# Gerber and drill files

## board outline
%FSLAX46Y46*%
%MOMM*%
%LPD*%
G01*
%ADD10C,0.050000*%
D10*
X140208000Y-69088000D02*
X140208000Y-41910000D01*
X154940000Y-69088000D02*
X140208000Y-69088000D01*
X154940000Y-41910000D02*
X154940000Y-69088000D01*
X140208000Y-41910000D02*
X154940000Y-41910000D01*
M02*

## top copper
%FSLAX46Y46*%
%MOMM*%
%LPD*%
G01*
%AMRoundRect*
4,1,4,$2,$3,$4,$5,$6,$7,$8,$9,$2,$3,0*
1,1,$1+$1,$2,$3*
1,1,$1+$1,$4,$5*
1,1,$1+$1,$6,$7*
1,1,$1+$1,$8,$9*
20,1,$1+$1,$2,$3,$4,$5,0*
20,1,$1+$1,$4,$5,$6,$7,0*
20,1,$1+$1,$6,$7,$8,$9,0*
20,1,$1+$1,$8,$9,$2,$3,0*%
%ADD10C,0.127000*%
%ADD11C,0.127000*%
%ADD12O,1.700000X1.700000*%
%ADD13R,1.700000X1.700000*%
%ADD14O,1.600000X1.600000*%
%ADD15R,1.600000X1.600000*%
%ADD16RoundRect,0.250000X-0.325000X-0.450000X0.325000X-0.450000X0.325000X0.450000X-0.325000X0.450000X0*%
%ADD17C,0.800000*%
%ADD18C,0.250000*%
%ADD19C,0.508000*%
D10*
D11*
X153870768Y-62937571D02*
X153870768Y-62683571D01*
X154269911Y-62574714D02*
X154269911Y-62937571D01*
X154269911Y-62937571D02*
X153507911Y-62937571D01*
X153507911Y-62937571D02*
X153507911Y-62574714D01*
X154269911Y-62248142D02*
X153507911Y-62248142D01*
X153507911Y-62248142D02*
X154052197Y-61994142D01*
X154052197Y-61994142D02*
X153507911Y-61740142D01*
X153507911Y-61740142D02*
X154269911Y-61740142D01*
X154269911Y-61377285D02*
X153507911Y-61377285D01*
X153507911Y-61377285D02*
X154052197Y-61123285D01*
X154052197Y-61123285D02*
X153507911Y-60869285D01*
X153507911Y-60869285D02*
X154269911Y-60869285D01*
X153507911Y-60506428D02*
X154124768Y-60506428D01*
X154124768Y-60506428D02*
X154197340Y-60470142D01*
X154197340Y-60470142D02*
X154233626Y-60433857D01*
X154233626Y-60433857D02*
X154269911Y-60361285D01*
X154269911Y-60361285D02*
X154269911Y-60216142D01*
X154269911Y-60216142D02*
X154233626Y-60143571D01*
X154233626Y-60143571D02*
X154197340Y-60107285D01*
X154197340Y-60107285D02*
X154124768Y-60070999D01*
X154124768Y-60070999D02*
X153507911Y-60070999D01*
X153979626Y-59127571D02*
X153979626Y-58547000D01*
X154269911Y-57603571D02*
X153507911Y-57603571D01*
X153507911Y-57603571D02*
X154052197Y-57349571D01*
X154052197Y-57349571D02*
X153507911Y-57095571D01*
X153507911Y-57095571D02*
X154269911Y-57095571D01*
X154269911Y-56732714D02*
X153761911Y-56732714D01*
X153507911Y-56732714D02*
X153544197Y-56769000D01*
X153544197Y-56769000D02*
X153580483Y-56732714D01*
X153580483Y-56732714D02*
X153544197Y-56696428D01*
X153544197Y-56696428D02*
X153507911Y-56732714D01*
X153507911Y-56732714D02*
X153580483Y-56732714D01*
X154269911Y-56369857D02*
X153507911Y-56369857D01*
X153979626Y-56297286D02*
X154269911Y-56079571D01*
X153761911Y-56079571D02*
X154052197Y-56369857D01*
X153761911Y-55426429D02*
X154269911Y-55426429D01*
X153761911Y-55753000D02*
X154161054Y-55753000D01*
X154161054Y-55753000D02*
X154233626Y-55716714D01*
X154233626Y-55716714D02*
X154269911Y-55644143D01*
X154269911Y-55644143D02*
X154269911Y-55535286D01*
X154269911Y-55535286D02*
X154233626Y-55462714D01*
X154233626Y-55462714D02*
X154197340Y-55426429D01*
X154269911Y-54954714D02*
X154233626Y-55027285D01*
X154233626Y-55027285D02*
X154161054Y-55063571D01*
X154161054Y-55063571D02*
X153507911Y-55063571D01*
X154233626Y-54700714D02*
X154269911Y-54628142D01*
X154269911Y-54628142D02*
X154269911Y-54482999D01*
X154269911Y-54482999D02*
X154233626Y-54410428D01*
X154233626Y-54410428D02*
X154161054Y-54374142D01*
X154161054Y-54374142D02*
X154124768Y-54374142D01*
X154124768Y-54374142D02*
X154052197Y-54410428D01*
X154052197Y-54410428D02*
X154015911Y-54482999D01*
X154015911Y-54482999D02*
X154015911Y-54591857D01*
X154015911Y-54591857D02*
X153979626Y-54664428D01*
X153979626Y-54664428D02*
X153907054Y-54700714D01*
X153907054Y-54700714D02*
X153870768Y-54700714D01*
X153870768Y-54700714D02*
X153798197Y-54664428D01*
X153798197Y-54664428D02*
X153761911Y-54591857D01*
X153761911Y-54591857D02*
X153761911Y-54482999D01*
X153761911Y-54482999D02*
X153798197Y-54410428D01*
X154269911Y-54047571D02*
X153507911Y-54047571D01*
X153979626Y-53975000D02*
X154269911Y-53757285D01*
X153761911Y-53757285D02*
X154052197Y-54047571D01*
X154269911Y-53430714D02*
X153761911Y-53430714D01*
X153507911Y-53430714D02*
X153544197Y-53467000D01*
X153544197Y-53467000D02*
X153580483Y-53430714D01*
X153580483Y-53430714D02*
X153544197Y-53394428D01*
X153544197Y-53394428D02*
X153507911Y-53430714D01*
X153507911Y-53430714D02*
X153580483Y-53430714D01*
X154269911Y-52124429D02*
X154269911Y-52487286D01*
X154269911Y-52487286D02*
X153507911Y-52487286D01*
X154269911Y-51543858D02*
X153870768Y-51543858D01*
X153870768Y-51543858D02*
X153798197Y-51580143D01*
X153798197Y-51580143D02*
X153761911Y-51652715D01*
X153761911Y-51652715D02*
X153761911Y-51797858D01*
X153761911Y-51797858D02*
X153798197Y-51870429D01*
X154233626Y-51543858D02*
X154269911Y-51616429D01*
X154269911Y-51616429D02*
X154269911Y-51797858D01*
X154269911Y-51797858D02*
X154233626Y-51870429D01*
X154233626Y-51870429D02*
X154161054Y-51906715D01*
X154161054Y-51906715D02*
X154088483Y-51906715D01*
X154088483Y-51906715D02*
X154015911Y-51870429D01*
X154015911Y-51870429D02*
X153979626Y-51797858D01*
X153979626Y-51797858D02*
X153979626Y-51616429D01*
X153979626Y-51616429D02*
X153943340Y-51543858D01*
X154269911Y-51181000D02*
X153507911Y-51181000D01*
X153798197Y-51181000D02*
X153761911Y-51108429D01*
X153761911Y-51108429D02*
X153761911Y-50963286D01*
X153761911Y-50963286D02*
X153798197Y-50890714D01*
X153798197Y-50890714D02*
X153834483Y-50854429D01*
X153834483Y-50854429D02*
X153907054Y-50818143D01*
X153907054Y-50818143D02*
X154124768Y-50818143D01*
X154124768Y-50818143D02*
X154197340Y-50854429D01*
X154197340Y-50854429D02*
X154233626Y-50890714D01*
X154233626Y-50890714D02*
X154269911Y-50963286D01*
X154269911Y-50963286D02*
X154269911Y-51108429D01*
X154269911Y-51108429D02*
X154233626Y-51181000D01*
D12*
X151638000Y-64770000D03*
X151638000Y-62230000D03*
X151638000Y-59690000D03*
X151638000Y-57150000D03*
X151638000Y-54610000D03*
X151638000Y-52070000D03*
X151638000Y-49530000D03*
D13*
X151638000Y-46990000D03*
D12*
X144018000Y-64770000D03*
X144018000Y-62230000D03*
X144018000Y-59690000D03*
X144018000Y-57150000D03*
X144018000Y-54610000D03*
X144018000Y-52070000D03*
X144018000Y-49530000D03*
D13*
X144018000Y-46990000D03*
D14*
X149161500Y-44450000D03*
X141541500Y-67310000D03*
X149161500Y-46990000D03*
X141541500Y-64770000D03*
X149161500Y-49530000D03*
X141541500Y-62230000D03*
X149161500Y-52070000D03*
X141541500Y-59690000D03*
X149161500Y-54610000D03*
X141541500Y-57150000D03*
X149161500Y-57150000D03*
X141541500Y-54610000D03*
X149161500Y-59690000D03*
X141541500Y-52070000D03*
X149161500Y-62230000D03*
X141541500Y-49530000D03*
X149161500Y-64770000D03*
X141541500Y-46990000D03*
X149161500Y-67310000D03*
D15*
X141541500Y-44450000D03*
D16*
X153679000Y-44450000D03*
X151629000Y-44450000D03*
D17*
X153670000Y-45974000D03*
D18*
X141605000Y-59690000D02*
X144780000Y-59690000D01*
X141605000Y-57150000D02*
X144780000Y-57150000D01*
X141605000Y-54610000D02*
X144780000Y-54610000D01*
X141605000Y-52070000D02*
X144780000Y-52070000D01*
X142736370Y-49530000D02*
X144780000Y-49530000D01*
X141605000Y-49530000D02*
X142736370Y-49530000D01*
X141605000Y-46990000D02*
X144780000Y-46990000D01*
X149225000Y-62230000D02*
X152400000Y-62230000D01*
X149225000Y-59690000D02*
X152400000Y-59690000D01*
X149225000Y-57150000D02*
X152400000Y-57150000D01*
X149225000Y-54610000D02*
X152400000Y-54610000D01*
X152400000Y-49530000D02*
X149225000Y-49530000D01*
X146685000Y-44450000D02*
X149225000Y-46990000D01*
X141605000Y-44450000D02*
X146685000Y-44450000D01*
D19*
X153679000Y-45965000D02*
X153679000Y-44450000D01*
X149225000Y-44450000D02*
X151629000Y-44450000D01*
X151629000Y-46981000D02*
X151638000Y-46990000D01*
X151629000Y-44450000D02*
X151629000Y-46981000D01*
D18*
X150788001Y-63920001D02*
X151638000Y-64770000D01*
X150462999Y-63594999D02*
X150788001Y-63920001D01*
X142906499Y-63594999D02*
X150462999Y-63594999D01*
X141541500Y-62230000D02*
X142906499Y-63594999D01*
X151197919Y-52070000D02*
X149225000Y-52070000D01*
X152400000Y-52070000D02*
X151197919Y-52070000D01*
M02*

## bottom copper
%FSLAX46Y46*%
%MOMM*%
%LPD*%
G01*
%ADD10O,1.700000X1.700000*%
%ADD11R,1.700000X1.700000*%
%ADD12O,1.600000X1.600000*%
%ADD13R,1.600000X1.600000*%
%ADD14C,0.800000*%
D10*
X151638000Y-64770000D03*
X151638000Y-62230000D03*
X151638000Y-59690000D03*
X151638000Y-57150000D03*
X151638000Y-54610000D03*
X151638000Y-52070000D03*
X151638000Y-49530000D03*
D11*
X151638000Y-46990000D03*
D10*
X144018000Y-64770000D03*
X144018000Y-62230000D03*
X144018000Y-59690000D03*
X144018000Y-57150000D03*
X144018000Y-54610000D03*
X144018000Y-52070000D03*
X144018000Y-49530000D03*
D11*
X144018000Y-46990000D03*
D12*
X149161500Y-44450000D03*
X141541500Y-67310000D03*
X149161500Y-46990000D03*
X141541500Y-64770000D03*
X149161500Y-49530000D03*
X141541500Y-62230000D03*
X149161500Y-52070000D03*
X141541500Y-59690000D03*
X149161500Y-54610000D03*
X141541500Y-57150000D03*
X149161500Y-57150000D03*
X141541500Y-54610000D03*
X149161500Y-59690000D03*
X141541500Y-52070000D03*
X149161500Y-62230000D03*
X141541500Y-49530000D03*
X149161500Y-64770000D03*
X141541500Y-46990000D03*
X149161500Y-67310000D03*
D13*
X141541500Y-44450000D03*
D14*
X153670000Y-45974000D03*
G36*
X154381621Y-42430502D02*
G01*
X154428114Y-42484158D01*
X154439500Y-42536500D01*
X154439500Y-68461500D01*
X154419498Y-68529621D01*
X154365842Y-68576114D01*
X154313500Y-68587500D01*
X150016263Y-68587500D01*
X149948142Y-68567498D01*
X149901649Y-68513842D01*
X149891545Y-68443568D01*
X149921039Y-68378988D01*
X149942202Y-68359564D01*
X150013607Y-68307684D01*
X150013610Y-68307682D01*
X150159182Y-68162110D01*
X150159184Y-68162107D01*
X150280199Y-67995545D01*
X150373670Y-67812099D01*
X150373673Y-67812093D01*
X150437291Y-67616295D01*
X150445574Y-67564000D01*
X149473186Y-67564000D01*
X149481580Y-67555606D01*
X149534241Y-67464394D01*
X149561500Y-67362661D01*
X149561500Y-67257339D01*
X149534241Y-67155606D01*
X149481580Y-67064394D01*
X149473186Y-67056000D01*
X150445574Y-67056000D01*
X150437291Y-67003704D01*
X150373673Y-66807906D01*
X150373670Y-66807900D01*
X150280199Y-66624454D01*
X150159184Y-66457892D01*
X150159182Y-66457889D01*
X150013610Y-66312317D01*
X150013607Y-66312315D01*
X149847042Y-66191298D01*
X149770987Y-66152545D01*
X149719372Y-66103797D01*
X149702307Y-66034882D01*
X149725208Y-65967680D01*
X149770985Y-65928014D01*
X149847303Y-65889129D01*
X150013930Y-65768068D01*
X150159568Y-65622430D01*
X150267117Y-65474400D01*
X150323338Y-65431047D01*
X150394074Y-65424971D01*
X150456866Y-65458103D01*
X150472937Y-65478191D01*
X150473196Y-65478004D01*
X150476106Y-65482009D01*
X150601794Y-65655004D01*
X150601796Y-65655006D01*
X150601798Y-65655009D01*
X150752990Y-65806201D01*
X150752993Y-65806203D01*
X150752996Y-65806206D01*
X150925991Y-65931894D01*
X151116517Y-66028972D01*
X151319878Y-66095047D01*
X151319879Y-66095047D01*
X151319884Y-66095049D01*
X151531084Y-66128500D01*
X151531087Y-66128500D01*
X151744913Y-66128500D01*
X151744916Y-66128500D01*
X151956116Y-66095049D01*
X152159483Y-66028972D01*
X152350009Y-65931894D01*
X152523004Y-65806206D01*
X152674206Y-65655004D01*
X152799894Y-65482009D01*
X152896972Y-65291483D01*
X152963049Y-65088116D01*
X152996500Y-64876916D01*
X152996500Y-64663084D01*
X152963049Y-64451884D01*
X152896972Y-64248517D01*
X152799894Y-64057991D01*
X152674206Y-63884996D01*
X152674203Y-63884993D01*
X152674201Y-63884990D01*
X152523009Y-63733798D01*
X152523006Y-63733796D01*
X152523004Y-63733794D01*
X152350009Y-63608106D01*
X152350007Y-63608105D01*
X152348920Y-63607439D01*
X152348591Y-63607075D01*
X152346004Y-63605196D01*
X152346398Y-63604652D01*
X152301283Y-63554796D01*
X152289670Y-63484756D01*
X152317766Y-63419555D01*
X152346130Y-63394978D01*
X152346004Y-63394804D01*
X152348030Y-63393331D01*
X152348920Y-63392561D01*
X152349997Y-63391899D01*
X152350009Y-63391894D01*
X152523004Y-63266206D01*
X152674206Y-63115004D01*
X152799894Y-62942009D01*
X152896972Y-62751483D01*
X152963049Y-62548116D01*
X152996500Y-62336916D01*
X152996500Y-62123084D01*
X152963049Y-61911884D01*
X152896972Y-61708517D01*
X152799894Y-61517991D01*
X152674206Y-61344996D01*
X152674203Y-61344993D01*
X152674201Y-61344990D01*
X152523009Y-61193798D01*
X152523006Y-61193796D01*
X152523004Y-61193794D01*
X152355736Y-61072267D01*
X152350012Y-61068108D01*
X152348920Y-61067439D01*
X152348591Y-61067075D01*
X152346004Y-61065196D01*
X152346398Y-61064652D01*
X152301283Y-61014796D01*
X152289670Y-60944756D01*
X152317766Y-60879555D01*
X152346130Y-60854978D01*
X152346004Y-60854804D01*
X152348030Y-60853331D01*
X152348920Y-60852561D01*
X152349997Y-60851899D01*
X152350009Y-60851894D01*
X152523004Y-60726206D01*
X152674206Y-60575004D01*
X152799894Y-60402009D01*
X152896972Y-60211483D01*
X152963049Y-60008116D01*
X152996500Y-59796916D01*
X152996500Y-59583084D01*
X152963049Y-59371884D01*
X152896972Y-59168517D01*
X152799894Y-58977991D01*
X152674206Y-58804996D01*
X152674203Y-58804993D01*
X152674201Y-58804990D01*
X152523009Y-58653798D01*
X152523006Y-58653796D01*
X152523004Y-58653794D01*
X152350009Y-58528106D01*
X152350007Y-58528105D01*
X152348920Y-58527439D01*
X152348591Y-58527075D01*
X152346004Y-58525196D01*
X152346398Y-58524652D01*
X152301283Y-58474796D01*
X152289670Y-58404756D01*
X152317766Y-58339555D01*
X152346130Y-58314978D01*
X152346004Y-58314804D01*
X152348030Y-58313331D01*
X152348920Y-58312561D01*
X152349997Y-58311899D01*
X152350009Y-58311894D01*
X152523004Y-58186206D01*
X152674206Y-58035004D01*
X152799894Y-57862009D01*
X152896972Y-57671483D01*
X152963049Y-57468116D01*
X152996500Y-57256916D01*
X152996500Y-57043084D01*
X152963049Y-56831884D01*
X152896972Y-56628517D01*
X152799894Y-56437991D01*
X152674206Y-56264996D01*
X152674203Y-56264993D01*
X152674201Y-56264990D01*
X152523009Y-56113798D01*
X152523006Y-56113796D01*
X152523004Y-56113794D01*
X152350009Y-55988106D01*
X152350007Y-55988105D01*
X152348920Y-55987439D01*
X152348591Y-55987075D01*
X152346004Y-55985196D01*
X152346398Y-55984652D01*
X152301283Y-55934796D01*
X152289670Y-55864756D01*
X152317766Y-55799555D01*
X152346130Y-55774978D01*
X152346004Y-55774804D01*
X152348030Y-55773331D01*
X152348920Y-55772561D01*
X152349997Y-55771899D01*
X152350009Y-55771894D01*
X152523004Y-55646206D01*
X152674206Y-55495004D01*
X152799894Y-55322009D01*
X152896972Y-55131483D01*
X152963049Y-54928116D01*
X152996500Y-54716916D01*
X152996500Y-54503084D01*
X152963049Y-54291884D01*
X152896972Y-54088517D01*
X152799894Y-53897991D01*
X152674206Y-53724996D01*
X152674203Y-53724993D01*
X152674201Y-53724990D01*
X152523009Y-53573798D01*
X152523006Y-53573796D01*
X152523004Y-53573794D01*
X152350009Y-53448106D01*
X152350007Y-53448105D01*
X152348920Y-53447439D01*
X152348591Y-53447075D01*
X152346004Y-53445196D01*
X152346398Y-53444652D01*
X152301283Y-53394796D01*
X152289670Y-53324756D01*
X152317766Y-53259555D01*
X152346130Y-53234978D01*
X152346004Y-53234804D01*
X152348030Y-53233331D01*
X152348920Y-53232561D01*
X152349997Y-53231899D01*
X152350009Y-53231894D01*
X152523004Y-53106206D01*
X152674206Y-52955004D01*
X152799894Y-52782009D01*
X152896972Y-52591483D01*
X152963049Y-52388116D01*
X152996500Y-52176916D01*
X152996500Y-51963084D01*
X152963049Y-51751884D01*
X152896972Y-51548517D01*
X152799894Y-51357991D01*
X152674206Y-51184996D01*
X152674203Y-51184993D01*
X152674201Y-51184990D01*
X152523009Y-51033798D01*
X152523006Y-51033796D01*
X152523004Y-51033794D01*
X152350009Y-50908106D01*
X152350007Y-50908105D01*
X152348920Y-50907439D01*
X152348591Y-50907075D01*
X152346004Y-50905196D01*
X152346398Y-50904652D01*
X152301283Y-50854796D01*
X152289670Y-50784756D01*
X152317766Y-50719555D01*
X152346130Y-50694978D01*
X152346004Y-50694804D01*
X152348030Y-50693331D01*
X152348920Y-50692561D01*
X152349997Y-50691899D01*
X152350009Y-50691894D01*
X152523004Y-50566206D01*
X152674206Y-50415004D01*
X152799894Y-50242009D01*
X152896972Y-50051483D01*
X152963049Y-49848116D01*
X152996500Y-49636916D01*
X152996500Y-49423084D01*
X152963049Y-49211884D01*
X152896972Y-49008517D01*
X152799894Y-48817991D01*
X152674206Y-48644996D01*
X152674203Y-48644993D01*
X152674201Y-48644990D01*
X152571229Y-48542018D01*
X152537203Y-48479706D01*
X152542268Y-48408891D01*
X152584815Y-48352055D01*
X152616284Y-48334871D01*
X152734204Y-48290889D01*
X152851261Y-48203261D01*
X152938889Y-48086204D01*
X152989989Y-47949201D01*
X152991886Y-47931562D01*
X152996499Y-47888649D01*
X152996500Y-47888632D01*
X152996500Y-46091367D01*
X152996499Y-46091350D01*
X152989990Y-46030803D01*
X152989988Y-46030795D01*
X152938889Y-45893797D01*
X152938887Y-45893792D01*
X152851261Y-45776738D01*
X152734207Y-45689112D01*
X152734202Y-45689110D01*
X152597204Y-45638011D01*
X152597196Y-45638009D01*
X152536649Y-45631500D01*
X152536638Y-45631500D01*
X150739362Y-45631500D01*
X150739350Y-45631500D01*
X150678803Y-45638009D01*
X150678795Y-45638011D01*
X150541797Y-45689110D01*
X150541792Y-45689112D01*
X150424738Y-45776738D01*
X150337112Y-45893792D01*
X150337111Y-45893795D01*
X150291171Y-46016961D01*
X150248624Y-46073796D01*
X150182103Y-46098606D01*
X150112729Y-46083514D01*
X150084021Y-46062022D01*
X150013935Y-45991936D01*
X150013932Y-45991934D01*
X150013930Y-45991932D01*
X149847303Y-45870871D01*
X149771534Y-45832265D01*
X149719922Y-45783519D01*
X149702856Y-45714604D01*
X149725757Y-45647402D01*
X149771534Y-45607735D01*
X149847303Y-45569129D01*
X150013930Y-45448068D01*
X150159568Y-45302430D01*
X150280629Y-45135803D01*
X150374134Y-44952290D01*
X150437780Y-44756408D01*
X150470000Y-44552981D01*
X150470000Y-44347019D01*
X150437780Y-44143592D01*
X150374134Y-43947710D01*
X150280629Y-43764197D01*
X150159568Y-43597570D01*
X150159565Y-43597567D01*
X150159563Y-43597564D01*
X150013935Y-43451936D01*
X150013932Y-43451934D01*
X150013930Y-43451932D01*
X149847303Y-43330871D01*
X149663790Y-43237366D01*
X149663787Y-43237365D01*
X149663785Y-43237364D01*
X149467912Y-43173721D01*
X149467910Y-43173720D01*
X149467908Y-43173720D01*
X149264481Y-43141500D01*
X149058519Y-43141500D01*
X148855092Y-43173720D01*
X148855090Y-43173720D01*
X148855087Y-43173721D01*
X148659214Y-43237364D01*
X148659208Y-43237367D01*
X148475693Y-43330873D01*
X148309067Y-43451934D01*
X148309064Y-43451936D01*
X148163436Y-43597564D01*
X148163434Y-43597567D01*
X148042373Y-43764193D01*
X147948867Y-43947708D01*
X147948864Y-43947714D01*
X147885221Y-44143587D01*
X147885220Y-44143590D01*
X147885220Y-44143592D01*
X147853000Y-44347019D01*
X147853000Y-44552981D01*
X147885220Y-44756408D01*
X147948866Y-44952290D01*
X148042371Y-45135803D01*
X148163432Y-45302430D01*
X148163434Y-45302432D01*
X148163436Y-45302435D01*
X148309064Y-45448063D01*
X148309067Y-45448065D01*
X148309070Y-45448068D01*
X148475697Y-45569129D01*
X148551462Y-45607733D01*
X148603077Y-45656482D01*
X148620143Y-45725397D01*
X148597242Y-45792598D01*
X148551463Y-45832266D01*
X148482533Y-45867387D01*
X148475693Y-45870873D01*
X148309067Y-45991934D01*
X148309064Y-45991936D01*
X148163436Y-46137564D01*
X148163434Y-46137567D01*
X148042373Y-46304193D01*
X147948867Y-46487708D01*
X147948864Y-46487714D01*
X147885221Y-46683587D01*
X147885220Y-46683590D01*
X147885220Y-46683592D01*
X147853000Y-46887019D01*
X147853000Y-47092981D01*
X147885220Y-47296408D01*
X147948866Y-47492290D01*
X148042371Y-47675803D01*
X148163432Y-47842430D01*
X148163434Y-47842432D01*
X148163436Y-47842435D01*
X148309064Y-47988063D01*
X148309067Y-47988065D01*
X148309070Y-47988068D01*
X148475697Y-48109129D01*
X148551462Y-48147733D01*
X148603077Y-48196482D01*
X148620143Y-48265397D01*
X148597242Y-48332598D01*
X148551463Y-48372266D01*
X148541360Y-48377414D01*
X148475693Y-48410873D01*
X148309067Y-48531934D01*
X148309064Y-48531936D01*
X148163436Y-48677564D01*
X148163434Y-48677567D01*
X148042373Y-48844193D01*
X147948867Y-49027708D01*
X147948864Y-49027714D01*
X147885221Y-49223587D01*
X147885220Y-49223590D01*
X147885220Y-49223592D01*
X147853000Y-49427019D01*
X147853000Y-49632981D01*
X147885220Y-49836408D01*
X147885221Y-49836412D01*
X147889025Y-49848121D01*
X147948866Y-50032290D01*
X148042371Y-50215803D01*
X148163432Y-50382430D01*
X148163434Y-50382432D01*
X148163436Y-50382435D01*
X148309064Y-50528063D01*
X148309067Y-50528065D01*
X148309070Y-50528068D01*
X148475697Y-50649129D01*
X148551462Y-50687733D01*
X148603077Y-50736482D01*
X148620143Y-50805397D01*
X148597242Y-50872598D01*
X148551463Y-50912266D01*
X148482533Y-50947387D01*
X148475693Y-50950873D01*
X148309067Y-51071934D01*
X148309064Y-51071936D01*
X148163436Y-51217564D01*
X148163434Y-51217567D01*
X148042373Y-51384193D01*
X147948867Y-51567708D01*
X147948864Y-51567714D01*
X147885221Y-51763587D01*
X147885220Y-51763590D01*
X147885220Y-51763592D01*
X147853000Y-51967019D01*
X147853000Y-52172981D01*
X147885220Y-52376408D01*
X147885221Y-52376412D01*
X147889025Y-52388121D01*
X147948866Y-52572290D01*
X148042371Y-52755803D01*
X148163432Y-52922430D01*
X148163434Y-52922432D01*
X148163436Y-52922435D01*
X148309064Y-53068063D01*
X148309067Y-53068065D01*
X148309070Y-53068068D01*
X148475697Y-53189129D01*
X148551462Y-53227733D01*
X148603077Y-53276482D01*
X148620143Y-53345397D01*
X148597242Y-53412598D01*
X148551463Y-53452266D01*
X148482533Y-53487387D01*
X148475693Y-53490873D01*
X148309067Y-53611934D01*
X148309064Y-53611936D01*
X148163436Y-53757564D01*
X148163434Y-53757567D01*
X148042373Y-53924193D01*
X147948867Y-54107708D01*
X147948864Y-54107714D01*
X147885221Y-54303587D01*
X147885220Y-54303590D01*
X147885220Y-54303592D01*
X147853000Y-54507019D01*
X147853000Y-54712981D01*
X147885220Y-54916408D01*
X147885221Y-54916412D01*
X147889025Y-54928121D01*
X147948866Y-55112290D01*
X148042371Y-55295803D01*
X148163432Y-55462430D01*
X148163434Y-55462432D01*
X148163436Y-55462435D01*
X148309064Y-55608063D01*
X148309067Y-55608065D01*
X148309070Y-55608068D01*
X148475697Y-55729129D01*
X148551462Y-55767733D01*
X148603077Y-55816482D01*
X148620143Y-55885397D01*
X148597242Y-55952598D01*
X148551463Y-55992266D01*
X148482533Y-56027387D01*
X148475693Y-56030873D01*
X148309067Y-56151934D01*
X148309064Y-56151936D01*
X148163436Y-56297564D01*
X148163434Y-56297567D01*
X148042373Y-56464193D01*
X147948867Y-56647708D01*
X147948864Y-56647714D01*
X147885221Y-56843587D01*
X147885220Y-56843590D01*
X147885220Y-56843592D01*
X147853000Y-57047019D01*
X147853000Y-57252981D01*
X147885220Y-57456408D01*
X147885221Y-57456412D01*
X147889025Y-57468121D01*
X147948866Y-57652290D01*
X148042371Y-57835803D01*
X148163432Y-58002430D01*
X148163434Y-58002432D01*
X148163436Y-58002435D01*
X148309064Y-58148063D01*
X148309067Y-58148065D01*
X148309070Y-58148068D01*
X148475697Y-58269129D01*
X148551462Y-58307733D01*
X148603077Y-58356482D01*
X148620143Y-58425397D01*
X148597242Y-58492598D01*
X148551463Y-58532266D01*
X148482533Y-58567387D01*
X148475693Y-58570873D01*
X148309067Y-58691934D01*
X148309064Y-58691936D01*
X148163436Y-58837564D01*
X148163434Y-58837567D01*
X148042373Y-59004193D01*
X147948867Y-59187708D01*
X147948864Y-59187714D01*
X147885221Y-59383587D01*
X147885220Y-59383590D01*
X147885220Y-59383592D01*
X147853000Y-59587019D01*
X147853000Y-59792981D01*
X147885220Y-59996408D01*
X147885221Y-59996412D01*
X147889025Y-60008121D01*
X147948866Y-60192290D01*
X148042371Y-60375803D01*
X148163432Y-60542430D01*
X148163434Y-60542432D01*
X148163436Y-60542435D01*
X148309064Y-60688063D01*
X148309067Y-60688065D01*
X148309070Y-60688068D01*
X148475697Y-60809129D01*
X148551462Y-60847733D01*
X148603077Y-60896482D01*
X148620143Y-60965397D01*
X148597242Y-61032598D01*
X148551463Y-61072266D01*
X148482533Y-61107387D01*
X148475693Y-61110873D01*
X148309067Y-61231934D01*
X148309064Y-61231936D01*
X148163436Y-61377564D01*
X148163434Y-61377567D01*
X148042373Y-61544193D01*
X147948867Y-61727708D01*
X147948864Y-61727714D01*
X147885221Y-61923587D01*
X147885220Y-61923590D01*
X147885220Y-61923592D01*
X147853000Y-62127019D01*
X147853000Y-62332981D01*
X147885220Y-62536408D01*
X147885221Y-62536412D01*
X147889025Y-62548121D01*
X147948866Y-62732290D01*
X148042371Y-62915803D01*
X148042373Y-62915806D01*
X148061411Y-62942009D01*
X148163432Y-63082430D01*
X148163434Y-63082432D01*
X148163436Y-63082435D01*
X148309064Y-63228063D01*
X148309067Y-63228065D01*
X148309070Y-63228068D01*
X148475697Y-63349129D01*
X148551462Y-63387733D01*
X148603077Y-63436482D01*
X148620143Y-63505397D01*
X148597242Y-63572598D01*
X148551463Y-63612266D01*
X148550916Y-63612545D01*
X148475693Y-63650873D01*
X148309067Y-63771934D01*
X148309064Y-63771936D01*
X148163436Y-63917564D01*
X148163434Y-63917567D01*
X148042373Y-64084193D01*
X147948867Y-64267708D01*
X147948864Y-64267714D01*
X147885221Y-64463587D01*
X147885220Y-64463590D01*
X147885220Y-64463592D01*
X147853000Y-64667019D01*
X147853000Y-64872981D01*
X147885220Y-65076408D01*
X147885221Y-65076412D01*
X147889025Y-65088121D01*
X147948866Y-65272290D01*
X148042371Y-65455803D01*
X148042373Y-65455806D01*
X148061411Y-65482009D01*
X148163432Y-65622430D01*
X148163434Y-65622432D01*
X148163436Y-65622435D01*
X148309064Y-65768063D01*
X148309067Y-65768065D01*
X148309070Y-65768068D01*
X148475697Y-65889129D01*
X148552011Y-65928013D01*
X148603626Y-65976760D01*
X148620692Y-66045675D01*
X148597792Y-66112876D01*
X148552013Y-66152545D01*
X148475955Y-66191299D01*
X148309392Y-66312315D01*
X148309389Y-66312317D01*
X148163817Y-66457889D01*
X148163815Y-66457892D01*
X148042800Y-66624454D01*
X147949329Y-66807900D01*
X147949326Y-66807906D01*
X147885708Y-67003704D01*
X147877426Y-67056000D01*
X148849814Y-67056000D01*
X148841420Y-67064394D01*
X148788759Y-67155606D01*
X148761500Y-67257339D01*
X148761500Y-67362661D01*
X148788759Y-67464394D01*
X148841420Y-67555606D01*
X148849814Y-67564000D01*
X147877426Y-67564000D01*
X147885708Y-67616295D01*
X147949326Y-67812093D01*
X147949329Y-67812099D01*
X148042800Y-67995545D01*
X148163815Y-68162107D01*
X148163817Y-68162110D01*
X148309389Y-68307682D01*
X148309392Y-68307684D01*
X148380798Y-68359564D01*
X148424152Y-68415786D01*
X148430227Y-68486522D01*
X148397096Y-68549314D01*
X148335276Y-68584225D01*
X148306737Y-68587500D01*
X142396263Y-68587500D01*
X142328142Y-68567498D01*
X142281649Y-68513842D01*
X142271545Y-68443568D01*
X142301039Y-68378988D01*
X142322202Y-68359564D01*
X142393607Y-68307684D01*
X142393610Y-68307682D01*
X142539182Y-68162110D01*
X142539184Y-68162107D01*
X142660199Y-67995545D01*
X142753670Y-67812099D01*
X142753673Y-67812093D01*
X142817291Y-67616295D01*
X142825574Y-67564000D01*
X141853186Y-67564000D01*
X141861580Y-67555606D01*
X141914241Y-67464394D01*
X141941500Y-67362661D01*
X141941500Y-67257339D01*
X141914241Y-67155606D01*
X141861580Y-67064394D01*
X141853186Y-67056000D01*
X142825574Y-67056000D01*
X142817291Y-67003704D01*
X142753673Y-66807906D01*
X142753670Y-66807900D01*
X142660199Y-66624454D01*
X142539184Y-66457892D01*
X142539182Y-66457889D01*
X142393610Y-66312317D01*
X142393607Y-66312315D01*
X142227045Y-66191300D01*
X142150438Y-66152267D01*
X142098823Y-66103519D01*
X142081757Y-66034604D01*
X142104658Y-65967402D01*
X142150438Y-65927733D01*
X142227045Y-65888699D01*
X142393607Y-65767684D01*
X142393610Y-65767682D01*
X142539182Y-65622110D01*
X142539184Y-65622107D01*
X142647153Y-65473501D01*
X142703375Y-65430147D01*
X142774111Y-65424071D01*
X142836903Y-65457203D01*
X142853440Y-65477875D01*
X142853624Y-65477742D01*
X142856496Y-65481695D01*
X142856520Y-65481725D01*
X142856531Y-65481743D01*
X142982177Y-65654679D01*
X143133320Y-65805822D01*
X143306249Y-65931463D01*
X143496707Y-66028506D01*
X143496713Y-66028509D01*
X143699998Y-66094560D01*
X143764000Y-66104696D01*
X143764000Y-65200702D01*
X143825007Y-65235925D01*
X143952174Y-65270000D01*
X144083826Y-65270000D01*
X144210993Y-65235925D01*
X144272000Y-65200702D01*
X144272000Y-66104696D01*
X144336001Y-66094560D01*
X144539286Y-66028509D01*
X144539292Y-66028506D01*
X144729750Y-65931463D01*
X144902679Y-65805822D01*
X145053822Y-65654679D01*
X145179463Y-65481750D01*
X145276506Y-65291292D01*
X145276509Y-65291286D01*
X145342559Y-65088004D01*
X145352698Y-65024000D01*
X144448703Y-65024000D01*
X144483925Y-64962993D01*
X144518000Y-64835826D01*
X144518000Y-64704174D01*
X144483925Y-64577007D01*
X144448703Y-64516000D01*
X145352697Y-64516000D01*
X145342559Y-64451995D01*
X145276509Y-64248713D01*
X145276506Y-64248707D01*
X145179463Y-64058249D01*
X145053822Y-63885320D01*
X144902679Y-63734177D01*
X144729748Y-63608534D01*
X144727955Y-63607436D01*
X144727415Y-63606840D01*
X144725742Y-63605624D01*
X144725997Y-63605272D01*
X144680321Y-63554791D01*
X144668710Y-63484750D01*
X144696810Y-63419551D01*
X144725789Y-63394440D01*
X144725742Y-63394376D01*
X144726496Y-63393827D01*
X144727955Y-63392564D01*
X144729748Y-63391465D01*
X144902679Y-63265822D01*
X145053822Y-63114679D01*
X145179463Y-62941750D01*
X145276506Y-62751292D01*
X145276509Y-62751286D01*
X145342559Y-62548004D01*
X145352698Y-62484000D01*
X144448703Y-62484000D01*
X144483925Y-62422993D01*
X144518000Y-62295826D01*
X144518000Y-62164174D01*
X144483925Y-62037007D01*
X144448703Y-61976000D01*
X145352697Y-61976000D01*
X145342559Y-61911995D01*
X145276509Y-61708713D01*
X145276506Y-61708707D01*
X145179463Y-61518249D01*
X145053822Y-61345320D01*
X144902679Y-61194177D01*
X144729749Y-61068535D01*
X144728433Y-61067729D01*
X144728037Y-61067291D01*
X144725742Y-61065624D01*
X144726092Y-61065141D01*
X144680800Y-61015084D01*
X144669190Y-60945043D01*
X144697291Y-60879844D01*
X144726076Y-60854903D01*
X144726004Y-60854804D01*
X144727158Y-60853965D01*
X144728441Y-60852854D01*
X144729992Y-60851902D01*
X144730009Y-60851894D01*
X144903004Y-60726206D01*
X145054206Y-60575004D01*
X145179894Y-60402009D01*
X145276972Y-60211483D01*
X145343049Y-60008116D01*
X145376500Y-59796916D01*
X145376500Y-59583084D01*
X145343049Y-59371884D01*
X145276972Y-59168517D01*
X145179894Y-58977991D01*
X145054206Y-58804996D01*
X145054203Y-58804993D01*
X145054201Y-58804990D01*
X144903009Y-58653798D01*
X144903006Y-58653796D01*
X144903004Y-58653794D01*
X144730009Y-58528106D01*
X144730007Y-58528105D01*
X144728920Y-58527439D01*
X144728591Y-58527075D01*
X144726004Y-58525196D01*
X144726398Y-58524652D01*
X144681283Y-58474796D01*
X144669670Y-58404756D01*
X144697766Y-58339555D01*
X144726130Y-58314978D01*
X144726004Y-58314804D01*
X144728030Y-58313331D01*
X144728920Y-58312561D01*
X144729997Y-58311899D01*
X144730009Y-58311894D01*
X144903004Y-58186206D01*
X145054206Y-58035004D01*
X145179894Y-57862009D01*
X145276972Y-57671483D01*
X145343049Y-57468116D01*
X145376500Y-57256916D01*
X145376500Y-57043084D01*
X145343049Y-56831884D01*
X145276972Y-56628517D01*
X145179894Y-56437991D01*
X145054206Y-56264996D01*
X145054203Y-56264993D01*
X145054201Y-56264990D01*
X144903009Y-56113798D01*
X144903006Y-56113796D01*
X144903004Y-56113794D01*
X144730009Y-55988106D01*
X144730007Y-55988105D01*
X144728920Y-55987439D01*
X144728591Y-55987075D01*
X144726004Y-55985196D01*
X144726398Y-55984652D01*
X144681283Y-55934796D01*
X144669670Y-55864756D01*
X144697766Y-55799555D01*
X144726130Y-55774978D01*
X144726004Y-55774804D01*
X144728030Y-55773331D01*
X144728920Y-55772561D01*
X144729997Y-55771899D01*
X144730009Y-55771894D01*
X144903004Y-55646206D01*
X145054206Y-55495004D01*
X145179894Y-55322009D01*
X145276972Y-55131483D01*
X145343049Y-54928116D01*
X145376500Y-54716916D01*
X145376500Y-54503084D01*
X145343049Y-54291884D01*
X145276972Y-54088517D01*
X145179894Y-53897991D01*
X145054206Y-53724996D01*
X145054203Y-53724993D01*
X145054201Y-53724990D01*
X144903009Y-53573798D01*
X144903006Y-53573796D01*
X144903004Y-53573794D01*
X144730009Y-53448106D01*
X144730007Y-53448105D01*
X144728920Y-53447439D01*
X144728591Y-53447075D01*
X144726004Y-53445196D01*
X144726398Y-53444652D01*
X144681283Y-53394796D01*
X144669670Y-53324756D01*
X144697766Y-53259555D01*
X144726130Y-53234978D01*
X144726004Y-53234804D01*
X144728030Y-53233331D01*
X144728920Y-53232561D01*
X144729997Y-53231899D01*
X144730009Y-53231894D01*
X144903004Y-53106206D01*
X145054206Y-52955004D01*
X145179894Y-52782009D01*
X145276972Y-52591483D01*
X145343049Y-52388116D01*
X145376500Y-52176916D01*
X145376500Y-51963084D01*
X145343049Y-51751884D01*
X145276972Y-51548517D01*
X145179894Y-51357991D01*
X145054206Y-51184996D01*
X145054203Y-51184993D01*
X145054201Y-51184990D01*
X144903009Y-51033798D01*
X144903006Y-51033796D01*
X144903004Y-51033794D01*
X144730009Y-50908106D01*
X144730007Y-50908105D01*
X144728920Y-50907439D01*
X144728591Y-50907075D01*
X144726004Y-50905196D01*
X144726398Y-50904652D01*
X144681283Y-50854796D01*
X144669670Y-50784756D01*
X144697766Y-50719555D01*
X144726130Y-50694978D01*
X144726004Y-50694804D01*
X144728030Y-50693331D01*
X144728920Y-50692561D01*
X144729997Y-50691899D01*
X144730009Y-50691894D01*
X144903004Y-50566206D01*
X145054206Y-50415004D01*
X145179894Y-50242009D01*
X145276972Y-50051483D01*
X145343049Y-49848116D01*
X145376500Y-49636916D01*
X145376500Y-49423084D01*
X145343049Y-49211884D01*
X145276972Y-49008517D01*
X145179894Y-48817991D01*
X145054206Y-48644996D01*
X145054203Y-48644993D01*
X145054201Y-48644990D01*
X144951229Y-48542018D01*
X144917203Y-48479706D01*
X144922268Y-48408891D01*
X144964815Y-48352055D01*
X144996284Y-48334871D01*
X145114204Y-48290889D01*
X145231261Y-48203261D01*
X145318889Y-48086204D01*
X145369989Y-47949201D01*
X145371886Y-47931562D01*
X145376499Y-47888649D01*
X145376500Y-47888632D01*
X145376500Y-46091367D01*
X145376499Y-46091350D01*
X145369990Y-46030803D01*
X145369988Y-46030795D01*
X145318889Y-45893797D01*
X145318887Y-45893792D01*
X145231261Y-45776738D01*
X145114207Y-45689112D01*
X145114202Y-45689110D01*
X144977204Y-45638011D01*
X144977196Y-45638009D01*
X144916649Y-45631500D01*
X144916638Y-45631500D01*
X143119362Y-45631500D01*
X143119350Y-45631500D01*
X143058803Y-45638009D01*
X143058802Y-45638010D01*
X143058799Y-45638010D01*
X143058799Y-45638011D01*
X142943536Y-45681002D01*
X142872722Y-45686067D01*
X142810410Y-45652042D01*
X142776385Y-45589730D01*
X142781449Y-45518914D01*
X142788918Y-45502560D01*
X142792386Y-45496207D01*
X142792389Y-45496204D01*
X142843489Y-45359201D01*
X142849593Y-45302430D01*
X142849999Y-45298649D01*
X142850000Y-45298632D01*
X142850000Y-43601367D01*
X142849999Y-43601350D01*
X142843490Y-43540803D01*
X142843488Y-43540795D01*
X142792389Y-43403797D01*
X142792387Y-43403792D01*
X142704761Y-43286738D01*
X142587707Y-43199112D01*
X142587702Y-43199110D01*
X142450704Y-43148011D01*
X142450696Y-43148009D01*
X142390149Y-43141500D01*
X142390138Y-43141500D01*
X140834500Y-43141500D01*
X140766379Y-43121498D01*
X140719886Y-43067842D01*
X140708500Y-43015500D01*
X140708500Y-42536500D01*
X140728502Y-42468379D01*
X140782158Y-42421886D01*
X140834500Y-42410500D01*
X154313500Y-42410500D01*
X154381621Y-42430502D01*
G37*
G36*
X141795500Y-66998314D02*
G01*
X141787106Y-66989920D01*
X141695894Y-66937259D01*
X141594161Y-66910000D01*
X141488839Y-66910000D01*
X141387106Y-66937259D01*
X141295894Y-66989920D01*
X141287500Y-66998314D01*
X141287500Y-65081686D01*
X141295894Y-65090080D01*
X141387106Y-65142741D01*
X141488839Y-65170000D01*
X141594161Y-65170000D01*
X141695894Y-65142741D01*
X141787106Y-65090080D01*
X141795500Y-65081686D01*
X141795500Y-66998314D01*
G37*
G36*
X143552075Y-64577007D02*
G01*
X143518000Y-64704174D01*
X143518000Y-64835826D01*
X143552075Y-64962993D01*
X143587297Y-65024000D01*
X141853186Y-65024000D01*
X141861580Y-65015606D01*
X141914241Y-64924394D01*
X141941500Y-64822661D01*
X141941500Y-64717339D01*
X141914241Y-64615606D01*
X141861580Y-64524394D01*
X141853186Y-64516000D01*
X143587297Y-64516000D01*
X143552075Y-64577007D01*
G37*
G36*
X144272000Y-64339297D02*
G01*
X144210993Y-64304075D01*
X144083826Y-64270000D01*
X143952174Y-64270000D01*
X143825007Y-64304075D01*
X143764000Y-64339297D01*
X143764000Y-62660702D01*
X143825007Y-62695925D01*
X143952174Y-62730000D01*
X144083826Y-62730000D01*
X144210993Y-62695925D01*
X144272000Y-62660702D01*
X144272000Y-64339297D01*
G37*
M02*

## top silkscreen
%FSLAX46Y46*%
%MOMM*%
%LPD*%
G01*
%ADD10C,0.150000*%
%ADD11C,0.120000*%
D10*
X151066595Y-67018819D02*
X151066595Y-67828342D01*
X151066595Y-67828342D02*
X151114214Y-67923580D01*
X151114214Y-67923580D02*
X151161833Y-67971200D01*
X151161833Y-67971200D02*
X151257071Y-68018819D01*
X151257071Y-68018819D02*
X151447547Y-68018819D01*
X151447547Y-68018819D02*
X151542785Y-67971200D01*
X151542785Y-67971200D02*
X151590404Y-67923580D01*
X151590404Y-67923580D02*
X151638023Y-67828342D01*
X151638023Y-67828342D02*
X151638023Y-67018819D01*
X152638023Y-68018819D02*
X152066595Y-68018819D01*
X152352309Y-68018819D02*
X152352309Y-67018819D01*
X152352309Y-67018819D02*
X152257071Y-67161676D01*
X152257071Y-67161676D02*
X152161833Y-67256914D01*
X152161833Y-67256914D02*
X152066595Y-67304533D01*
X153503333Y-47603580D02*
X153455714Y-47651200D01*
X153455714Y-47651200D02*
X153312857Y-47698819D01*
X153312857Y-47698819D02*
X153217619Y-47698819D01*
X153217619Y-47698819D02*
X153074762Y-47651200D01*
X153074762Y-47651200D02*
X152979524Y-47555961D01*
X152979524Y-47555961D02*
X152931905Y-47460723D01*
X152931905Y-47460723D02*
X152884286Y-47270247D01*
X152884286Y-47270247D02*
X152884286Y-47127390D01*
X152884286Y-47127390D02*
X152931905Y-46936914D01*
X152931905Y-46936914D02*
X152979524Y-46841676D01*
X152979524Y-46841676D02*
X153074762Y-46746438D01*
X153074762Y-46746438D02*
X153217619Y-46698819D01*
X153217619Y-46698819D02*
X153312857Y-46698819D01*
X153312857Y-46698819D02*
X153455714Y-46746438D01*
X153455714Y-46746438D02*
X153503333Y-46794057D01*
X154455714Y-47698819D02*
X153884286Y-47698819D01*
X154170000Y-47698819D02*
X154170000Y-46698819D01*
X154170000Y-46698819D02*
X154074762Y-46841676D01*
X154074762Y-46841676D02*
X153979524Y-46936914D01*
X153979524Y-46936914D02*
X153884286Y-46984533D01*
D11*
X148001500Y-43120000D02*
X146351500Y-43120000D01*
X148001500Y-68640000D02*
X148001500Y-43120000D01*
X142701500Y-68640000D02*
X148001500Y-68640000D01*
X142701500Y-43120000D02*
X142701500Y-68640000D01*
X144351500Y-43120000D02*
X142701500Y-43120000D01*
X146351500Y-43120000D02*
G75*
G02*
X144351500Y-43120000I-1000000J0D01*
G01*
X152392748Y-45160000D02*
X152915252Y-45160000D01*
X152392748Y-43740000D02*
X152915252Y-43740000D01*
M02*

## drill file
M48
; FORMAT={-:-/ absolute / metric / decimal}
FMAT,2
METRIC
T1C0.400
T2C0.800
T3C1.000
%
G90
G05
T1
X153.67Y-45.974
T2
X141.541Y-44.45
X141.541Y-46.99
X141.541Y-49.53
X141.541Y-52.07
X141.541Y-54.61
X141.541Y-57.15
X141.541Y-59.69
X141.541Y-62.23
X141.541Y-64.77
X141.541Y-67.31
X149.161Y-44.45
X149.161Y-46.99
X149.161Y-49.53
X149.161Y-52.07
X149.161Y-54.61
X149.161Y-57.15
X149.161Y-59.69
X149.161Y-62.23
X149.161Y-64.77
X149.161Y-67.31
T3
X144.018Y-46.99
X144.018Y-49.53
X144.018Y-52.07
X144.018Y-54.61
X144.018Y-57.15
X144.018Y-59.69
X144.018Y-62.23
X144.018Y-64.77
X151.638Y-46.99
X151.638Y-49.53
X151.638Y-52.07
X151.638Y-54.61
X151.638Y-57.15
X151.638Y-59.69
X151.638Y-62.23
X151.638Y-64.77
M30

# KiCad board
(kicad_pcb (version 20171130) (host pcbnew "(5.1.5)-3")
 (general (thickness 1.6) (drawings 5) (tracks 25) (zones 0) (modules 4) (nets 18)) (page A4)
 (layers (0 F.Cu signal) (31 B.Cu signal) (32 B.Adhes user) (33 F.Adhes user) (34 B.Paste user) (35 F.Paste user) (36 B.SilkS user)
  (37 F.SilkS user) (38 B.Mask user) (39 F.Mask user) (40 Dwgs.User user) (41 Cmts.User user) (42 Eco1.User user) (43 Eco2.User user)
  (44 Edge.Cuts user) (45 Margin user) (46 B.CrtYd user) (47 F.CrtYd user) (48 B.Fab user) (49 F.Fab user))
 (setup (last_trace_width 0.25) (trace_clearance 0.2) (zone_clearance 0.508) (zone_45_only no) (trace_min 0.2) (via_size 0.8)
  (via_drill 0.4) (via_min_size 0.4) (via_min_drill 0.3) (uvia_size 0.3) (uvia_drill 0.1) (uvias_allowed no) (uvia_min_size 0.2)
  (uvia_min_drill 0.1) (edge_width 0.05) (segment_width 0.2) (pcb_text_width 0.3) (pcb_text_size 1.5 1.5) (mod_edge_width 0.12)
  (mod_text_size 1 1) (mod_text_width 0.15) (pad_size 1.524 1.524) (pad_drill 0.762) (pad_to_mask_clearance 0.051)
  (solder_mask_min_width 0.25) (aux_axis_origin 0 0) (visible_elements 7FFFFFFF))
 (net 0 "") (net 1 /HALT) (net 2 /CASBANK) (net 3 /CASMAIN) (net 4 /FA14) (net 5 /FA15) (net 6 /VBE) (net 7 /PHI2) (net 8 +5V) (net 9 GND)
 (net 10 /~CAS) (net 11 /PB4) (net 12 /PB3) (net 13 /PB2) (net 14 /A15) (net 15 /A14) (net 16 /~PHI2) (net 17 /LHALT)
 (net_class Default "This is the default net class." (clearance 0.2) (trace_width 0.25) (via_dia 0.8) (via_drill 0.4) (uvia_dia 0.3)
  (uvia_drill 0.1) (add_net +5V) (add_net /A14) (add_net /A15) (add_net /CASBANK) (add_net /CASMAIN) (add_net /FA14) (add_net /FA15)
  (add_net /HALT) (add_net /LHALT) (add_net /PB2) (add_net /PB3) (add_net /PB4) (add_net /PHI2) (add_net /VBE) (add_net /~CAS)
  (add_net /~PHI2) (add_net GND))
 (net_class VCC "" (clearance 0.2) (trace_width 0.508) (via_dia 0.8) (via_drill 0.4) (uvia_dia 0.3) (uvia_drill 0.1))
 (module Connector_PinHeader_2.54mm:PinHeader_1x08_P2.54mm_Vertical (layer B.Cu) (at 151.638 46.99 180)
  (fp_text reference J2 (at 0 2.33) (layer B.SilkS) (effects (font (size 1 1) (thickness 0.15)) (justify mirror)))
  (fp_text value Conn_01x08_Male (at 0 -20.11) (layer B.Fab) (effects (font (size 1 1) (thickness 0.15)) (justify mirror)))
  (pad 8 thru_hole oval (at 0 -17.78 180) (size 1.7 1.7) (drill 1) (layers *.Cu *.Mask) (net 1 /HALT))
  (pad 7 thru_hole oval (at 0 -15.24 180) (size 1.7 1.7) (drill 1) (layers *.Cu *.Mask) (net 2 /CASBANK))
  (pad 6 thru_hole oval (at 0 -12.7 180) (size 1.7 1.7) (drill 1) (layers *.Cu *.Mask) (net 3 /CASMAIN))
  (pad 5 thru_hole oval (at 0 -10.16 180) (size 1.7 1.7) (drill 1) (layers *.Cu *.Mask) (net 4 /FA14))
  (pad 4 thru_hole oval (at 0 -7.62 180) (size 1.7 1.7) (drill 1) (layers *.Cu *.Mask) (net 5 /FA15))
  (pad 3 thru_hole oval (at 0 -5.08 180) (size 1.7 1.7) (drill 1) (layers *.Cu *.Mask) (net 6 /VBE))
  (pad 2 thru_hole oval (at 0 -2.54 180) (size 1.7 1.7) (drill 1) (layers *.Cu *.Mask) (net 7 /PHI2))
  (pad 1 thru_hole rect (at 0 0 180) (size 1.7 1.7) (drill 1) (layers *.Cu *.Mask) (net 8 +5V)))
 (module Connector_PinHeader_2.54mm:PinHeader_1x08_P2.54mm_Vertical (layer B.Cu) (at 144.018 46.99 180)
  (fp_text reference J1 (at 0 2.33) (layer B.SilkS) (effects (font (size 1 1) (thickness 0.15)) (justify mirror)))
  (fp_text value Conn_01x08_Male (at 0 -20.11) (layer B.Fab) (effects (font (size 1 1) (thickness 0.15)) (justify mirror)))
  (pad 8 thru_hole oval (at 0 -17.78 180) (size 1.7 1.7) (drill 1) (layers *.Cu *.Mask) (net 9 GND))
  (pad 7 thru_hole oval (at 0 -15.24 180) (size 1.7 1.7) (drill 1) (layers *.Cu *.Mask) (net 9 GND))
  (pad 6 thru_hole oval (at 0 -12.7 180) (size 1.7 1.7) (drill 1) (layers *.Cu *.Mask) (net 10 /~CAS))
  (pad 5 thru_hole oval (at 0 -10.16 180) (size 1.7 1.7) (drill 1) (layers *.Cu *.Mask) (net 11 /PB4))
  (pad 4 thru_hole oval (at 0 -7.62 180) (size 1.7 1.7) (drill 1) (layers *.Cu *.Mask) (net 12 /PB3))
  (pad 3 thru_hole oval (at 0 -5.08 180) (size 1.7 1.7) (drill 1) (layers *.Cu *.Mask) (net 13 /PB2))
  (pad 2 thru_hole oval (at 0 -2.54 180) (size 1.7 1.7) (drill 1) (layers *.Cu *.Mask) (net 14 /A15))
  (pad 1 thru_hole rect (at 0 0 180) (size 1.7 1.7) (drill 1) (layers *.Cu *.Mask) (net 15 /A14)))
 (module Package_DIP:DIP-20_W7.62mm (layer F.Cu) (at 141.5415 44.45)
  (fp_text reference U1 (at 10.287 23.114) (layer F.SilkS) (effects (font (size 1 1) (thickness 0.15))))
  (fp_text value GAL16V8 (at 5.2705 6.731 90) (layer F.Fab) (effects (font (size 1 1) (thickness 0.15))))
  (fp_line (start 6.46 -1.33) (end 4.81 -1.33) (layer F.SilkS) (width 0.12))
  (fp_line (start 6.46 24.19) (end 6.46 -1.33) (layer F.SilkS) (width 0.12))
  (fp_line (start 1.16 24.19) (end 6.46 24.19) (layer F.SilkS) (width 0.12))
  (fp_line (start 1.16 -1.33) (end 1.16 24.19) (layer F.SilkS) (width 0.12))
  (fp_line (start 2.81 -1.33) (end 1.16 -1.33) (layer F.SilkS) (width 0.12))
  (fp_arc (start 3.81 -1.33) (end 2.81 -1.33) (angle -180) (layer F.SilkS) (width 0.12))
  (pad 20 thru_hole oval (at 7.62 0) (size 1.6 1.6) (drill 0.8) (layers *.Cu *.Mask) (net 8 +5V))
  (pad 10 thru_hole oval (at 0 22.86) (size 1.6 1.6) (drill 0.8) (layers *.Cu *.Mask) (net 9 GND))
  (pad 19 thru_hole oval (at 7.62 2.54) (size 1.6 1.6) (drill 0.8) (layers *.Cu *.Mask) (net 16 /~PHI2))
  (pad 9 thru_hole oval (at 0 20.32) (size 1.6 1.6) (drill 0.8) (layers *.Cu *.Mask) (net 9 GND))
  (pad 18 thru_hole oval (at 7.62 5.08) (size 1.6 1.6) (drill 0.8) (layers *.Cu *.Mask) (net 7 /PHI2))
  (pad 8 thru_hole oval (at 0 17.78) (size 1.6 1.6) (drill 0.8) (layers *.Cu *.Mask) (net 1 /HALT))
  (pad 17 thru_hole oval (at 7.62 7.62) (size 1.6 1.6) (drill 0.8) (layers *.Cu *.Mask) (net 6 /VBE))
  (pad 7 thru_hole oval (at 0 15.24) (size 1.6 1.6) (drill 0.8) (layers *.Cu *.Mask) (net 10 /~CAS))
  (pad 16 thru_hole oval (at 7.62 10.16) (size 1.6 1.6) (drill 0.8) (layers *.Cu *.Mask) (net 5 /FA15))
  (pad 6 thru_hole oval (at 0 12.7) (size 1.6 1.6) (drill 0.8) (layers *.Cu *.Mask) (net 11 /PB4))
  (pad 15 thru_hole oval (at 7.62 12.7) (size 1.6 1.6) (drill 0.8) (layers *.Cu *.Mask) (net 4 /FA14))
  (pad 5 thru_hole oval (at 0 10.16) (size 1.6 1.6) (drill 0.8) (layers *.Cu *.Mask) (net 12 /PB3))
  (pad 14 thru_hole oval (at 7.62 15.24) (size 1.6 1.6) (drill 0.8) (layers *.Cu *.Mask) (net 3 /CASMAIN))
  (pad 4 thru_hole oval (at 0 7.62) (size 1.6 1.6) (drill 0.8) (layers *.Cu *.Mask) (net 13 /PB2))
  (pad 13 thru_hole oval (at 7.62 17.78) (size 1.6 1.6) (drill 0.8) (layers *.Cu *.Mask) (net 2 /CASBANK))
  (pad 3 thru_hole oval (at 0 5.08) (size 1.6 1.6) (drill 0.8) (layers *.Cu *.Mask) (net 14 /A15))
  (pad 12 thru_hole oval (at 7.62 20.32) (size 1.6 1.6) (drill 0.8) (layers *.Cu *.Mask) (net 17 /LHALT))
  (pad 2 thru_hole oval (at 0 2.54) (size 1.6 1.6) (drill 0.8) (layers *.Cu *.Mask) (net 15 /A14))
  (pad 11 thru_hole oval (at 7.62 22.86) (size 1.6 1.6) (drill 0.8) (layers *.Cu *.Mask) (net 9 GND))
  (pad 1 thru_hole rect (at 0 0) (size 1.6 1.6) (drill 0.8) (layers *.Cu *.Mask) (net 16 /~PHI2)))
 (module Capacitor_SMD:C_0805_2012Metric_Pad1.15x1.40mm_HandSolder (layer F.Cu) (at 152.654 44.45)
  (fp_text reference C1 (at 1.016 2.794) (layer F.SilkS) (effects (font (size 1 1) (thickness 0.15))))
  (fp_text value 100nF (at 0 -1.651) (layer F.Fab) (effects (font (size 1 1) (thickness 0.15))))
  (fp_line (start -0.261252 0.71) (end 0.261252 0.71) (layer F.SilkS) (width 0.12))
  (fp_line (start -0.261252 -0.71) (end 0.261252 -0.71) (layer F.SilkS) (width 0.12))
  (pad 2 smd roundrect (at 1.025 0) (size 1.15 1.4) (layers F.Cu F.Paste F.Mask) (roundrect_rratio 0.217391) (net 9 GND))
  (pad 1 smd roundrect (at -1.025 0) (size 1.15 1.4) (layers F.Cu F.Paste F.Mask) (roundrect_rratio 0.217391) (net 8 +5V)))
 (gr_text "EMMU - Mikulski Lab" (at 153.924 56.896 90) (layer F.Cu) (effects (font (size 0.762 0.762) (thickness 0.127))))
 (gr_line (start 140.208 69.088) (end 140.208 41.91) (layer Edge.Cuts) (width 0.05))
 (gr_line (start 154.94 69.088) (end 140.208 69.088) (layer Edge.Cuts) (width 0.05))
 (gr_line (start 154.94 41.91) (end 154.94 69.088) (layer Edge.Cuts) (width 0.05))
 (gr_line (start 140.208 41.91) (end 154.94 41.91) (layer Edge.Cuts) (width 0.05))
 (segment (start 141.605 59.69) (end 144.78 59.69) (width 0.25) (layer F.Cu) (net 10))
 (segment (start 141.605 57.15) (end 144.78 57.15) (width 0.25) (layer F.Cu) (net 11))
 (segment (start 141.605 54.61) (end 144.78 54.61) (width 0.25) (layer F.Cu) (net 12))
 (segment (start 141.605 52.07) (end 144.78 52.07) (width 0.25) (layer F.Cu) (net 13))
 (segment (start 142.73637 49.53) (end 144.78 49.53) (width 0.25) (layer F.Cu) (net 14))
 (segment (start 141.605 49.53) (end 142.73637 49.53) (width 0.25) (layer F.Cu) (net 14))
 (segment (start 141.605 46.99) (end 144.78 46.99) (width 0.25) (layer F.Cu) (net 15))
 (segment (start 149.225 62.23) (end 152.4 62.23) (width 0.25) (layer F.Cu) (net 2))
 (segment (start 149.225 59.69) (end 152.4 59.69) (width 0.25) (layer F.Cu) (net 3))
 (segment (start 149.225 57.15) (end 152.4 57.15) (width 0.25) (layer F.Cu) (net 4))
 (segment (start 149.225 54.61) (end 152.4 54.61) (width 0.25) (layer F.Cu) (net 5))
 (segment (start 152.4 49.53) (end 149.225 49.53) (width 0.25) (layer F.Cu) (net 7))
 (segment (start 146.685 44.45) (end 149.225 46.99) (width 0.25) (layer F.Cu) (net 16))
 (segment (start 141.605 44.45) (end 146.685 44.45) (width 0.25) (layer F.Cu) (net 16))
 (segment (start 153.679 45.965) (end 153.679 44.45) (width 0.508) (layer F.Cu) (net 9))
 (via (at 153.67 45.974) (size 0.8) (drill 0.4) (layers F.Cu B.Cu) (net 9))
 (segment (start 149.225 44.45) (end 151.629 44.45) (width 0.508) (layer F.Cu) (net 8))
 (segment (start 151.629 46.981) (end 151.638 46.99) (width 0.508) (layer F.Cu) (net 8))
 (segment (start 151.629 44.45) (end 151.629 46.981) (width 0.508) (layer F.Cu) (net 8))
 (segment (start 150.788001 63.920001) (end 151.638 64.77) (width 0.25) (layer F.Cu) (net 1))
 (segment (start 150.462999 63.594999) (end 150.788001 63.920001) (width 0.25) (layer F.Cu) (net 1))
 (segment (start 142.906499 63.594999) (end 150.462999 63.594999) (width 0.25) (layer F.Cu) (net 1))
 (segment (start 141.5415 62.23) (end 142.906499 63.594999) (width 0.25) (layer F.Cu) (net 1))
 (segment (start 151.197919 52.07) (end 149.225 52.07) (width 0.25) (layer F.Cu) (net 6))
 (segment (start 152.4 52.07) (end 151.197919 52.07) (width 0.25) (layer F.Cu) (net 6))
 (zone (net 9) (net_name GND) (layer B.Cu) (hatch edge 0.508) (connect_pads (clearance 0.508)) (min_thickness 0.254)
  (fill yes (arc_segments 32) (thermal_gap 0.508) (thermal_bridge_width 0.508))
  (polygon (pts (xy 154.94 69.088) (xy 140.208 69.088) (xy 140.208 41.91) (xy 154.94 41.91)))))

